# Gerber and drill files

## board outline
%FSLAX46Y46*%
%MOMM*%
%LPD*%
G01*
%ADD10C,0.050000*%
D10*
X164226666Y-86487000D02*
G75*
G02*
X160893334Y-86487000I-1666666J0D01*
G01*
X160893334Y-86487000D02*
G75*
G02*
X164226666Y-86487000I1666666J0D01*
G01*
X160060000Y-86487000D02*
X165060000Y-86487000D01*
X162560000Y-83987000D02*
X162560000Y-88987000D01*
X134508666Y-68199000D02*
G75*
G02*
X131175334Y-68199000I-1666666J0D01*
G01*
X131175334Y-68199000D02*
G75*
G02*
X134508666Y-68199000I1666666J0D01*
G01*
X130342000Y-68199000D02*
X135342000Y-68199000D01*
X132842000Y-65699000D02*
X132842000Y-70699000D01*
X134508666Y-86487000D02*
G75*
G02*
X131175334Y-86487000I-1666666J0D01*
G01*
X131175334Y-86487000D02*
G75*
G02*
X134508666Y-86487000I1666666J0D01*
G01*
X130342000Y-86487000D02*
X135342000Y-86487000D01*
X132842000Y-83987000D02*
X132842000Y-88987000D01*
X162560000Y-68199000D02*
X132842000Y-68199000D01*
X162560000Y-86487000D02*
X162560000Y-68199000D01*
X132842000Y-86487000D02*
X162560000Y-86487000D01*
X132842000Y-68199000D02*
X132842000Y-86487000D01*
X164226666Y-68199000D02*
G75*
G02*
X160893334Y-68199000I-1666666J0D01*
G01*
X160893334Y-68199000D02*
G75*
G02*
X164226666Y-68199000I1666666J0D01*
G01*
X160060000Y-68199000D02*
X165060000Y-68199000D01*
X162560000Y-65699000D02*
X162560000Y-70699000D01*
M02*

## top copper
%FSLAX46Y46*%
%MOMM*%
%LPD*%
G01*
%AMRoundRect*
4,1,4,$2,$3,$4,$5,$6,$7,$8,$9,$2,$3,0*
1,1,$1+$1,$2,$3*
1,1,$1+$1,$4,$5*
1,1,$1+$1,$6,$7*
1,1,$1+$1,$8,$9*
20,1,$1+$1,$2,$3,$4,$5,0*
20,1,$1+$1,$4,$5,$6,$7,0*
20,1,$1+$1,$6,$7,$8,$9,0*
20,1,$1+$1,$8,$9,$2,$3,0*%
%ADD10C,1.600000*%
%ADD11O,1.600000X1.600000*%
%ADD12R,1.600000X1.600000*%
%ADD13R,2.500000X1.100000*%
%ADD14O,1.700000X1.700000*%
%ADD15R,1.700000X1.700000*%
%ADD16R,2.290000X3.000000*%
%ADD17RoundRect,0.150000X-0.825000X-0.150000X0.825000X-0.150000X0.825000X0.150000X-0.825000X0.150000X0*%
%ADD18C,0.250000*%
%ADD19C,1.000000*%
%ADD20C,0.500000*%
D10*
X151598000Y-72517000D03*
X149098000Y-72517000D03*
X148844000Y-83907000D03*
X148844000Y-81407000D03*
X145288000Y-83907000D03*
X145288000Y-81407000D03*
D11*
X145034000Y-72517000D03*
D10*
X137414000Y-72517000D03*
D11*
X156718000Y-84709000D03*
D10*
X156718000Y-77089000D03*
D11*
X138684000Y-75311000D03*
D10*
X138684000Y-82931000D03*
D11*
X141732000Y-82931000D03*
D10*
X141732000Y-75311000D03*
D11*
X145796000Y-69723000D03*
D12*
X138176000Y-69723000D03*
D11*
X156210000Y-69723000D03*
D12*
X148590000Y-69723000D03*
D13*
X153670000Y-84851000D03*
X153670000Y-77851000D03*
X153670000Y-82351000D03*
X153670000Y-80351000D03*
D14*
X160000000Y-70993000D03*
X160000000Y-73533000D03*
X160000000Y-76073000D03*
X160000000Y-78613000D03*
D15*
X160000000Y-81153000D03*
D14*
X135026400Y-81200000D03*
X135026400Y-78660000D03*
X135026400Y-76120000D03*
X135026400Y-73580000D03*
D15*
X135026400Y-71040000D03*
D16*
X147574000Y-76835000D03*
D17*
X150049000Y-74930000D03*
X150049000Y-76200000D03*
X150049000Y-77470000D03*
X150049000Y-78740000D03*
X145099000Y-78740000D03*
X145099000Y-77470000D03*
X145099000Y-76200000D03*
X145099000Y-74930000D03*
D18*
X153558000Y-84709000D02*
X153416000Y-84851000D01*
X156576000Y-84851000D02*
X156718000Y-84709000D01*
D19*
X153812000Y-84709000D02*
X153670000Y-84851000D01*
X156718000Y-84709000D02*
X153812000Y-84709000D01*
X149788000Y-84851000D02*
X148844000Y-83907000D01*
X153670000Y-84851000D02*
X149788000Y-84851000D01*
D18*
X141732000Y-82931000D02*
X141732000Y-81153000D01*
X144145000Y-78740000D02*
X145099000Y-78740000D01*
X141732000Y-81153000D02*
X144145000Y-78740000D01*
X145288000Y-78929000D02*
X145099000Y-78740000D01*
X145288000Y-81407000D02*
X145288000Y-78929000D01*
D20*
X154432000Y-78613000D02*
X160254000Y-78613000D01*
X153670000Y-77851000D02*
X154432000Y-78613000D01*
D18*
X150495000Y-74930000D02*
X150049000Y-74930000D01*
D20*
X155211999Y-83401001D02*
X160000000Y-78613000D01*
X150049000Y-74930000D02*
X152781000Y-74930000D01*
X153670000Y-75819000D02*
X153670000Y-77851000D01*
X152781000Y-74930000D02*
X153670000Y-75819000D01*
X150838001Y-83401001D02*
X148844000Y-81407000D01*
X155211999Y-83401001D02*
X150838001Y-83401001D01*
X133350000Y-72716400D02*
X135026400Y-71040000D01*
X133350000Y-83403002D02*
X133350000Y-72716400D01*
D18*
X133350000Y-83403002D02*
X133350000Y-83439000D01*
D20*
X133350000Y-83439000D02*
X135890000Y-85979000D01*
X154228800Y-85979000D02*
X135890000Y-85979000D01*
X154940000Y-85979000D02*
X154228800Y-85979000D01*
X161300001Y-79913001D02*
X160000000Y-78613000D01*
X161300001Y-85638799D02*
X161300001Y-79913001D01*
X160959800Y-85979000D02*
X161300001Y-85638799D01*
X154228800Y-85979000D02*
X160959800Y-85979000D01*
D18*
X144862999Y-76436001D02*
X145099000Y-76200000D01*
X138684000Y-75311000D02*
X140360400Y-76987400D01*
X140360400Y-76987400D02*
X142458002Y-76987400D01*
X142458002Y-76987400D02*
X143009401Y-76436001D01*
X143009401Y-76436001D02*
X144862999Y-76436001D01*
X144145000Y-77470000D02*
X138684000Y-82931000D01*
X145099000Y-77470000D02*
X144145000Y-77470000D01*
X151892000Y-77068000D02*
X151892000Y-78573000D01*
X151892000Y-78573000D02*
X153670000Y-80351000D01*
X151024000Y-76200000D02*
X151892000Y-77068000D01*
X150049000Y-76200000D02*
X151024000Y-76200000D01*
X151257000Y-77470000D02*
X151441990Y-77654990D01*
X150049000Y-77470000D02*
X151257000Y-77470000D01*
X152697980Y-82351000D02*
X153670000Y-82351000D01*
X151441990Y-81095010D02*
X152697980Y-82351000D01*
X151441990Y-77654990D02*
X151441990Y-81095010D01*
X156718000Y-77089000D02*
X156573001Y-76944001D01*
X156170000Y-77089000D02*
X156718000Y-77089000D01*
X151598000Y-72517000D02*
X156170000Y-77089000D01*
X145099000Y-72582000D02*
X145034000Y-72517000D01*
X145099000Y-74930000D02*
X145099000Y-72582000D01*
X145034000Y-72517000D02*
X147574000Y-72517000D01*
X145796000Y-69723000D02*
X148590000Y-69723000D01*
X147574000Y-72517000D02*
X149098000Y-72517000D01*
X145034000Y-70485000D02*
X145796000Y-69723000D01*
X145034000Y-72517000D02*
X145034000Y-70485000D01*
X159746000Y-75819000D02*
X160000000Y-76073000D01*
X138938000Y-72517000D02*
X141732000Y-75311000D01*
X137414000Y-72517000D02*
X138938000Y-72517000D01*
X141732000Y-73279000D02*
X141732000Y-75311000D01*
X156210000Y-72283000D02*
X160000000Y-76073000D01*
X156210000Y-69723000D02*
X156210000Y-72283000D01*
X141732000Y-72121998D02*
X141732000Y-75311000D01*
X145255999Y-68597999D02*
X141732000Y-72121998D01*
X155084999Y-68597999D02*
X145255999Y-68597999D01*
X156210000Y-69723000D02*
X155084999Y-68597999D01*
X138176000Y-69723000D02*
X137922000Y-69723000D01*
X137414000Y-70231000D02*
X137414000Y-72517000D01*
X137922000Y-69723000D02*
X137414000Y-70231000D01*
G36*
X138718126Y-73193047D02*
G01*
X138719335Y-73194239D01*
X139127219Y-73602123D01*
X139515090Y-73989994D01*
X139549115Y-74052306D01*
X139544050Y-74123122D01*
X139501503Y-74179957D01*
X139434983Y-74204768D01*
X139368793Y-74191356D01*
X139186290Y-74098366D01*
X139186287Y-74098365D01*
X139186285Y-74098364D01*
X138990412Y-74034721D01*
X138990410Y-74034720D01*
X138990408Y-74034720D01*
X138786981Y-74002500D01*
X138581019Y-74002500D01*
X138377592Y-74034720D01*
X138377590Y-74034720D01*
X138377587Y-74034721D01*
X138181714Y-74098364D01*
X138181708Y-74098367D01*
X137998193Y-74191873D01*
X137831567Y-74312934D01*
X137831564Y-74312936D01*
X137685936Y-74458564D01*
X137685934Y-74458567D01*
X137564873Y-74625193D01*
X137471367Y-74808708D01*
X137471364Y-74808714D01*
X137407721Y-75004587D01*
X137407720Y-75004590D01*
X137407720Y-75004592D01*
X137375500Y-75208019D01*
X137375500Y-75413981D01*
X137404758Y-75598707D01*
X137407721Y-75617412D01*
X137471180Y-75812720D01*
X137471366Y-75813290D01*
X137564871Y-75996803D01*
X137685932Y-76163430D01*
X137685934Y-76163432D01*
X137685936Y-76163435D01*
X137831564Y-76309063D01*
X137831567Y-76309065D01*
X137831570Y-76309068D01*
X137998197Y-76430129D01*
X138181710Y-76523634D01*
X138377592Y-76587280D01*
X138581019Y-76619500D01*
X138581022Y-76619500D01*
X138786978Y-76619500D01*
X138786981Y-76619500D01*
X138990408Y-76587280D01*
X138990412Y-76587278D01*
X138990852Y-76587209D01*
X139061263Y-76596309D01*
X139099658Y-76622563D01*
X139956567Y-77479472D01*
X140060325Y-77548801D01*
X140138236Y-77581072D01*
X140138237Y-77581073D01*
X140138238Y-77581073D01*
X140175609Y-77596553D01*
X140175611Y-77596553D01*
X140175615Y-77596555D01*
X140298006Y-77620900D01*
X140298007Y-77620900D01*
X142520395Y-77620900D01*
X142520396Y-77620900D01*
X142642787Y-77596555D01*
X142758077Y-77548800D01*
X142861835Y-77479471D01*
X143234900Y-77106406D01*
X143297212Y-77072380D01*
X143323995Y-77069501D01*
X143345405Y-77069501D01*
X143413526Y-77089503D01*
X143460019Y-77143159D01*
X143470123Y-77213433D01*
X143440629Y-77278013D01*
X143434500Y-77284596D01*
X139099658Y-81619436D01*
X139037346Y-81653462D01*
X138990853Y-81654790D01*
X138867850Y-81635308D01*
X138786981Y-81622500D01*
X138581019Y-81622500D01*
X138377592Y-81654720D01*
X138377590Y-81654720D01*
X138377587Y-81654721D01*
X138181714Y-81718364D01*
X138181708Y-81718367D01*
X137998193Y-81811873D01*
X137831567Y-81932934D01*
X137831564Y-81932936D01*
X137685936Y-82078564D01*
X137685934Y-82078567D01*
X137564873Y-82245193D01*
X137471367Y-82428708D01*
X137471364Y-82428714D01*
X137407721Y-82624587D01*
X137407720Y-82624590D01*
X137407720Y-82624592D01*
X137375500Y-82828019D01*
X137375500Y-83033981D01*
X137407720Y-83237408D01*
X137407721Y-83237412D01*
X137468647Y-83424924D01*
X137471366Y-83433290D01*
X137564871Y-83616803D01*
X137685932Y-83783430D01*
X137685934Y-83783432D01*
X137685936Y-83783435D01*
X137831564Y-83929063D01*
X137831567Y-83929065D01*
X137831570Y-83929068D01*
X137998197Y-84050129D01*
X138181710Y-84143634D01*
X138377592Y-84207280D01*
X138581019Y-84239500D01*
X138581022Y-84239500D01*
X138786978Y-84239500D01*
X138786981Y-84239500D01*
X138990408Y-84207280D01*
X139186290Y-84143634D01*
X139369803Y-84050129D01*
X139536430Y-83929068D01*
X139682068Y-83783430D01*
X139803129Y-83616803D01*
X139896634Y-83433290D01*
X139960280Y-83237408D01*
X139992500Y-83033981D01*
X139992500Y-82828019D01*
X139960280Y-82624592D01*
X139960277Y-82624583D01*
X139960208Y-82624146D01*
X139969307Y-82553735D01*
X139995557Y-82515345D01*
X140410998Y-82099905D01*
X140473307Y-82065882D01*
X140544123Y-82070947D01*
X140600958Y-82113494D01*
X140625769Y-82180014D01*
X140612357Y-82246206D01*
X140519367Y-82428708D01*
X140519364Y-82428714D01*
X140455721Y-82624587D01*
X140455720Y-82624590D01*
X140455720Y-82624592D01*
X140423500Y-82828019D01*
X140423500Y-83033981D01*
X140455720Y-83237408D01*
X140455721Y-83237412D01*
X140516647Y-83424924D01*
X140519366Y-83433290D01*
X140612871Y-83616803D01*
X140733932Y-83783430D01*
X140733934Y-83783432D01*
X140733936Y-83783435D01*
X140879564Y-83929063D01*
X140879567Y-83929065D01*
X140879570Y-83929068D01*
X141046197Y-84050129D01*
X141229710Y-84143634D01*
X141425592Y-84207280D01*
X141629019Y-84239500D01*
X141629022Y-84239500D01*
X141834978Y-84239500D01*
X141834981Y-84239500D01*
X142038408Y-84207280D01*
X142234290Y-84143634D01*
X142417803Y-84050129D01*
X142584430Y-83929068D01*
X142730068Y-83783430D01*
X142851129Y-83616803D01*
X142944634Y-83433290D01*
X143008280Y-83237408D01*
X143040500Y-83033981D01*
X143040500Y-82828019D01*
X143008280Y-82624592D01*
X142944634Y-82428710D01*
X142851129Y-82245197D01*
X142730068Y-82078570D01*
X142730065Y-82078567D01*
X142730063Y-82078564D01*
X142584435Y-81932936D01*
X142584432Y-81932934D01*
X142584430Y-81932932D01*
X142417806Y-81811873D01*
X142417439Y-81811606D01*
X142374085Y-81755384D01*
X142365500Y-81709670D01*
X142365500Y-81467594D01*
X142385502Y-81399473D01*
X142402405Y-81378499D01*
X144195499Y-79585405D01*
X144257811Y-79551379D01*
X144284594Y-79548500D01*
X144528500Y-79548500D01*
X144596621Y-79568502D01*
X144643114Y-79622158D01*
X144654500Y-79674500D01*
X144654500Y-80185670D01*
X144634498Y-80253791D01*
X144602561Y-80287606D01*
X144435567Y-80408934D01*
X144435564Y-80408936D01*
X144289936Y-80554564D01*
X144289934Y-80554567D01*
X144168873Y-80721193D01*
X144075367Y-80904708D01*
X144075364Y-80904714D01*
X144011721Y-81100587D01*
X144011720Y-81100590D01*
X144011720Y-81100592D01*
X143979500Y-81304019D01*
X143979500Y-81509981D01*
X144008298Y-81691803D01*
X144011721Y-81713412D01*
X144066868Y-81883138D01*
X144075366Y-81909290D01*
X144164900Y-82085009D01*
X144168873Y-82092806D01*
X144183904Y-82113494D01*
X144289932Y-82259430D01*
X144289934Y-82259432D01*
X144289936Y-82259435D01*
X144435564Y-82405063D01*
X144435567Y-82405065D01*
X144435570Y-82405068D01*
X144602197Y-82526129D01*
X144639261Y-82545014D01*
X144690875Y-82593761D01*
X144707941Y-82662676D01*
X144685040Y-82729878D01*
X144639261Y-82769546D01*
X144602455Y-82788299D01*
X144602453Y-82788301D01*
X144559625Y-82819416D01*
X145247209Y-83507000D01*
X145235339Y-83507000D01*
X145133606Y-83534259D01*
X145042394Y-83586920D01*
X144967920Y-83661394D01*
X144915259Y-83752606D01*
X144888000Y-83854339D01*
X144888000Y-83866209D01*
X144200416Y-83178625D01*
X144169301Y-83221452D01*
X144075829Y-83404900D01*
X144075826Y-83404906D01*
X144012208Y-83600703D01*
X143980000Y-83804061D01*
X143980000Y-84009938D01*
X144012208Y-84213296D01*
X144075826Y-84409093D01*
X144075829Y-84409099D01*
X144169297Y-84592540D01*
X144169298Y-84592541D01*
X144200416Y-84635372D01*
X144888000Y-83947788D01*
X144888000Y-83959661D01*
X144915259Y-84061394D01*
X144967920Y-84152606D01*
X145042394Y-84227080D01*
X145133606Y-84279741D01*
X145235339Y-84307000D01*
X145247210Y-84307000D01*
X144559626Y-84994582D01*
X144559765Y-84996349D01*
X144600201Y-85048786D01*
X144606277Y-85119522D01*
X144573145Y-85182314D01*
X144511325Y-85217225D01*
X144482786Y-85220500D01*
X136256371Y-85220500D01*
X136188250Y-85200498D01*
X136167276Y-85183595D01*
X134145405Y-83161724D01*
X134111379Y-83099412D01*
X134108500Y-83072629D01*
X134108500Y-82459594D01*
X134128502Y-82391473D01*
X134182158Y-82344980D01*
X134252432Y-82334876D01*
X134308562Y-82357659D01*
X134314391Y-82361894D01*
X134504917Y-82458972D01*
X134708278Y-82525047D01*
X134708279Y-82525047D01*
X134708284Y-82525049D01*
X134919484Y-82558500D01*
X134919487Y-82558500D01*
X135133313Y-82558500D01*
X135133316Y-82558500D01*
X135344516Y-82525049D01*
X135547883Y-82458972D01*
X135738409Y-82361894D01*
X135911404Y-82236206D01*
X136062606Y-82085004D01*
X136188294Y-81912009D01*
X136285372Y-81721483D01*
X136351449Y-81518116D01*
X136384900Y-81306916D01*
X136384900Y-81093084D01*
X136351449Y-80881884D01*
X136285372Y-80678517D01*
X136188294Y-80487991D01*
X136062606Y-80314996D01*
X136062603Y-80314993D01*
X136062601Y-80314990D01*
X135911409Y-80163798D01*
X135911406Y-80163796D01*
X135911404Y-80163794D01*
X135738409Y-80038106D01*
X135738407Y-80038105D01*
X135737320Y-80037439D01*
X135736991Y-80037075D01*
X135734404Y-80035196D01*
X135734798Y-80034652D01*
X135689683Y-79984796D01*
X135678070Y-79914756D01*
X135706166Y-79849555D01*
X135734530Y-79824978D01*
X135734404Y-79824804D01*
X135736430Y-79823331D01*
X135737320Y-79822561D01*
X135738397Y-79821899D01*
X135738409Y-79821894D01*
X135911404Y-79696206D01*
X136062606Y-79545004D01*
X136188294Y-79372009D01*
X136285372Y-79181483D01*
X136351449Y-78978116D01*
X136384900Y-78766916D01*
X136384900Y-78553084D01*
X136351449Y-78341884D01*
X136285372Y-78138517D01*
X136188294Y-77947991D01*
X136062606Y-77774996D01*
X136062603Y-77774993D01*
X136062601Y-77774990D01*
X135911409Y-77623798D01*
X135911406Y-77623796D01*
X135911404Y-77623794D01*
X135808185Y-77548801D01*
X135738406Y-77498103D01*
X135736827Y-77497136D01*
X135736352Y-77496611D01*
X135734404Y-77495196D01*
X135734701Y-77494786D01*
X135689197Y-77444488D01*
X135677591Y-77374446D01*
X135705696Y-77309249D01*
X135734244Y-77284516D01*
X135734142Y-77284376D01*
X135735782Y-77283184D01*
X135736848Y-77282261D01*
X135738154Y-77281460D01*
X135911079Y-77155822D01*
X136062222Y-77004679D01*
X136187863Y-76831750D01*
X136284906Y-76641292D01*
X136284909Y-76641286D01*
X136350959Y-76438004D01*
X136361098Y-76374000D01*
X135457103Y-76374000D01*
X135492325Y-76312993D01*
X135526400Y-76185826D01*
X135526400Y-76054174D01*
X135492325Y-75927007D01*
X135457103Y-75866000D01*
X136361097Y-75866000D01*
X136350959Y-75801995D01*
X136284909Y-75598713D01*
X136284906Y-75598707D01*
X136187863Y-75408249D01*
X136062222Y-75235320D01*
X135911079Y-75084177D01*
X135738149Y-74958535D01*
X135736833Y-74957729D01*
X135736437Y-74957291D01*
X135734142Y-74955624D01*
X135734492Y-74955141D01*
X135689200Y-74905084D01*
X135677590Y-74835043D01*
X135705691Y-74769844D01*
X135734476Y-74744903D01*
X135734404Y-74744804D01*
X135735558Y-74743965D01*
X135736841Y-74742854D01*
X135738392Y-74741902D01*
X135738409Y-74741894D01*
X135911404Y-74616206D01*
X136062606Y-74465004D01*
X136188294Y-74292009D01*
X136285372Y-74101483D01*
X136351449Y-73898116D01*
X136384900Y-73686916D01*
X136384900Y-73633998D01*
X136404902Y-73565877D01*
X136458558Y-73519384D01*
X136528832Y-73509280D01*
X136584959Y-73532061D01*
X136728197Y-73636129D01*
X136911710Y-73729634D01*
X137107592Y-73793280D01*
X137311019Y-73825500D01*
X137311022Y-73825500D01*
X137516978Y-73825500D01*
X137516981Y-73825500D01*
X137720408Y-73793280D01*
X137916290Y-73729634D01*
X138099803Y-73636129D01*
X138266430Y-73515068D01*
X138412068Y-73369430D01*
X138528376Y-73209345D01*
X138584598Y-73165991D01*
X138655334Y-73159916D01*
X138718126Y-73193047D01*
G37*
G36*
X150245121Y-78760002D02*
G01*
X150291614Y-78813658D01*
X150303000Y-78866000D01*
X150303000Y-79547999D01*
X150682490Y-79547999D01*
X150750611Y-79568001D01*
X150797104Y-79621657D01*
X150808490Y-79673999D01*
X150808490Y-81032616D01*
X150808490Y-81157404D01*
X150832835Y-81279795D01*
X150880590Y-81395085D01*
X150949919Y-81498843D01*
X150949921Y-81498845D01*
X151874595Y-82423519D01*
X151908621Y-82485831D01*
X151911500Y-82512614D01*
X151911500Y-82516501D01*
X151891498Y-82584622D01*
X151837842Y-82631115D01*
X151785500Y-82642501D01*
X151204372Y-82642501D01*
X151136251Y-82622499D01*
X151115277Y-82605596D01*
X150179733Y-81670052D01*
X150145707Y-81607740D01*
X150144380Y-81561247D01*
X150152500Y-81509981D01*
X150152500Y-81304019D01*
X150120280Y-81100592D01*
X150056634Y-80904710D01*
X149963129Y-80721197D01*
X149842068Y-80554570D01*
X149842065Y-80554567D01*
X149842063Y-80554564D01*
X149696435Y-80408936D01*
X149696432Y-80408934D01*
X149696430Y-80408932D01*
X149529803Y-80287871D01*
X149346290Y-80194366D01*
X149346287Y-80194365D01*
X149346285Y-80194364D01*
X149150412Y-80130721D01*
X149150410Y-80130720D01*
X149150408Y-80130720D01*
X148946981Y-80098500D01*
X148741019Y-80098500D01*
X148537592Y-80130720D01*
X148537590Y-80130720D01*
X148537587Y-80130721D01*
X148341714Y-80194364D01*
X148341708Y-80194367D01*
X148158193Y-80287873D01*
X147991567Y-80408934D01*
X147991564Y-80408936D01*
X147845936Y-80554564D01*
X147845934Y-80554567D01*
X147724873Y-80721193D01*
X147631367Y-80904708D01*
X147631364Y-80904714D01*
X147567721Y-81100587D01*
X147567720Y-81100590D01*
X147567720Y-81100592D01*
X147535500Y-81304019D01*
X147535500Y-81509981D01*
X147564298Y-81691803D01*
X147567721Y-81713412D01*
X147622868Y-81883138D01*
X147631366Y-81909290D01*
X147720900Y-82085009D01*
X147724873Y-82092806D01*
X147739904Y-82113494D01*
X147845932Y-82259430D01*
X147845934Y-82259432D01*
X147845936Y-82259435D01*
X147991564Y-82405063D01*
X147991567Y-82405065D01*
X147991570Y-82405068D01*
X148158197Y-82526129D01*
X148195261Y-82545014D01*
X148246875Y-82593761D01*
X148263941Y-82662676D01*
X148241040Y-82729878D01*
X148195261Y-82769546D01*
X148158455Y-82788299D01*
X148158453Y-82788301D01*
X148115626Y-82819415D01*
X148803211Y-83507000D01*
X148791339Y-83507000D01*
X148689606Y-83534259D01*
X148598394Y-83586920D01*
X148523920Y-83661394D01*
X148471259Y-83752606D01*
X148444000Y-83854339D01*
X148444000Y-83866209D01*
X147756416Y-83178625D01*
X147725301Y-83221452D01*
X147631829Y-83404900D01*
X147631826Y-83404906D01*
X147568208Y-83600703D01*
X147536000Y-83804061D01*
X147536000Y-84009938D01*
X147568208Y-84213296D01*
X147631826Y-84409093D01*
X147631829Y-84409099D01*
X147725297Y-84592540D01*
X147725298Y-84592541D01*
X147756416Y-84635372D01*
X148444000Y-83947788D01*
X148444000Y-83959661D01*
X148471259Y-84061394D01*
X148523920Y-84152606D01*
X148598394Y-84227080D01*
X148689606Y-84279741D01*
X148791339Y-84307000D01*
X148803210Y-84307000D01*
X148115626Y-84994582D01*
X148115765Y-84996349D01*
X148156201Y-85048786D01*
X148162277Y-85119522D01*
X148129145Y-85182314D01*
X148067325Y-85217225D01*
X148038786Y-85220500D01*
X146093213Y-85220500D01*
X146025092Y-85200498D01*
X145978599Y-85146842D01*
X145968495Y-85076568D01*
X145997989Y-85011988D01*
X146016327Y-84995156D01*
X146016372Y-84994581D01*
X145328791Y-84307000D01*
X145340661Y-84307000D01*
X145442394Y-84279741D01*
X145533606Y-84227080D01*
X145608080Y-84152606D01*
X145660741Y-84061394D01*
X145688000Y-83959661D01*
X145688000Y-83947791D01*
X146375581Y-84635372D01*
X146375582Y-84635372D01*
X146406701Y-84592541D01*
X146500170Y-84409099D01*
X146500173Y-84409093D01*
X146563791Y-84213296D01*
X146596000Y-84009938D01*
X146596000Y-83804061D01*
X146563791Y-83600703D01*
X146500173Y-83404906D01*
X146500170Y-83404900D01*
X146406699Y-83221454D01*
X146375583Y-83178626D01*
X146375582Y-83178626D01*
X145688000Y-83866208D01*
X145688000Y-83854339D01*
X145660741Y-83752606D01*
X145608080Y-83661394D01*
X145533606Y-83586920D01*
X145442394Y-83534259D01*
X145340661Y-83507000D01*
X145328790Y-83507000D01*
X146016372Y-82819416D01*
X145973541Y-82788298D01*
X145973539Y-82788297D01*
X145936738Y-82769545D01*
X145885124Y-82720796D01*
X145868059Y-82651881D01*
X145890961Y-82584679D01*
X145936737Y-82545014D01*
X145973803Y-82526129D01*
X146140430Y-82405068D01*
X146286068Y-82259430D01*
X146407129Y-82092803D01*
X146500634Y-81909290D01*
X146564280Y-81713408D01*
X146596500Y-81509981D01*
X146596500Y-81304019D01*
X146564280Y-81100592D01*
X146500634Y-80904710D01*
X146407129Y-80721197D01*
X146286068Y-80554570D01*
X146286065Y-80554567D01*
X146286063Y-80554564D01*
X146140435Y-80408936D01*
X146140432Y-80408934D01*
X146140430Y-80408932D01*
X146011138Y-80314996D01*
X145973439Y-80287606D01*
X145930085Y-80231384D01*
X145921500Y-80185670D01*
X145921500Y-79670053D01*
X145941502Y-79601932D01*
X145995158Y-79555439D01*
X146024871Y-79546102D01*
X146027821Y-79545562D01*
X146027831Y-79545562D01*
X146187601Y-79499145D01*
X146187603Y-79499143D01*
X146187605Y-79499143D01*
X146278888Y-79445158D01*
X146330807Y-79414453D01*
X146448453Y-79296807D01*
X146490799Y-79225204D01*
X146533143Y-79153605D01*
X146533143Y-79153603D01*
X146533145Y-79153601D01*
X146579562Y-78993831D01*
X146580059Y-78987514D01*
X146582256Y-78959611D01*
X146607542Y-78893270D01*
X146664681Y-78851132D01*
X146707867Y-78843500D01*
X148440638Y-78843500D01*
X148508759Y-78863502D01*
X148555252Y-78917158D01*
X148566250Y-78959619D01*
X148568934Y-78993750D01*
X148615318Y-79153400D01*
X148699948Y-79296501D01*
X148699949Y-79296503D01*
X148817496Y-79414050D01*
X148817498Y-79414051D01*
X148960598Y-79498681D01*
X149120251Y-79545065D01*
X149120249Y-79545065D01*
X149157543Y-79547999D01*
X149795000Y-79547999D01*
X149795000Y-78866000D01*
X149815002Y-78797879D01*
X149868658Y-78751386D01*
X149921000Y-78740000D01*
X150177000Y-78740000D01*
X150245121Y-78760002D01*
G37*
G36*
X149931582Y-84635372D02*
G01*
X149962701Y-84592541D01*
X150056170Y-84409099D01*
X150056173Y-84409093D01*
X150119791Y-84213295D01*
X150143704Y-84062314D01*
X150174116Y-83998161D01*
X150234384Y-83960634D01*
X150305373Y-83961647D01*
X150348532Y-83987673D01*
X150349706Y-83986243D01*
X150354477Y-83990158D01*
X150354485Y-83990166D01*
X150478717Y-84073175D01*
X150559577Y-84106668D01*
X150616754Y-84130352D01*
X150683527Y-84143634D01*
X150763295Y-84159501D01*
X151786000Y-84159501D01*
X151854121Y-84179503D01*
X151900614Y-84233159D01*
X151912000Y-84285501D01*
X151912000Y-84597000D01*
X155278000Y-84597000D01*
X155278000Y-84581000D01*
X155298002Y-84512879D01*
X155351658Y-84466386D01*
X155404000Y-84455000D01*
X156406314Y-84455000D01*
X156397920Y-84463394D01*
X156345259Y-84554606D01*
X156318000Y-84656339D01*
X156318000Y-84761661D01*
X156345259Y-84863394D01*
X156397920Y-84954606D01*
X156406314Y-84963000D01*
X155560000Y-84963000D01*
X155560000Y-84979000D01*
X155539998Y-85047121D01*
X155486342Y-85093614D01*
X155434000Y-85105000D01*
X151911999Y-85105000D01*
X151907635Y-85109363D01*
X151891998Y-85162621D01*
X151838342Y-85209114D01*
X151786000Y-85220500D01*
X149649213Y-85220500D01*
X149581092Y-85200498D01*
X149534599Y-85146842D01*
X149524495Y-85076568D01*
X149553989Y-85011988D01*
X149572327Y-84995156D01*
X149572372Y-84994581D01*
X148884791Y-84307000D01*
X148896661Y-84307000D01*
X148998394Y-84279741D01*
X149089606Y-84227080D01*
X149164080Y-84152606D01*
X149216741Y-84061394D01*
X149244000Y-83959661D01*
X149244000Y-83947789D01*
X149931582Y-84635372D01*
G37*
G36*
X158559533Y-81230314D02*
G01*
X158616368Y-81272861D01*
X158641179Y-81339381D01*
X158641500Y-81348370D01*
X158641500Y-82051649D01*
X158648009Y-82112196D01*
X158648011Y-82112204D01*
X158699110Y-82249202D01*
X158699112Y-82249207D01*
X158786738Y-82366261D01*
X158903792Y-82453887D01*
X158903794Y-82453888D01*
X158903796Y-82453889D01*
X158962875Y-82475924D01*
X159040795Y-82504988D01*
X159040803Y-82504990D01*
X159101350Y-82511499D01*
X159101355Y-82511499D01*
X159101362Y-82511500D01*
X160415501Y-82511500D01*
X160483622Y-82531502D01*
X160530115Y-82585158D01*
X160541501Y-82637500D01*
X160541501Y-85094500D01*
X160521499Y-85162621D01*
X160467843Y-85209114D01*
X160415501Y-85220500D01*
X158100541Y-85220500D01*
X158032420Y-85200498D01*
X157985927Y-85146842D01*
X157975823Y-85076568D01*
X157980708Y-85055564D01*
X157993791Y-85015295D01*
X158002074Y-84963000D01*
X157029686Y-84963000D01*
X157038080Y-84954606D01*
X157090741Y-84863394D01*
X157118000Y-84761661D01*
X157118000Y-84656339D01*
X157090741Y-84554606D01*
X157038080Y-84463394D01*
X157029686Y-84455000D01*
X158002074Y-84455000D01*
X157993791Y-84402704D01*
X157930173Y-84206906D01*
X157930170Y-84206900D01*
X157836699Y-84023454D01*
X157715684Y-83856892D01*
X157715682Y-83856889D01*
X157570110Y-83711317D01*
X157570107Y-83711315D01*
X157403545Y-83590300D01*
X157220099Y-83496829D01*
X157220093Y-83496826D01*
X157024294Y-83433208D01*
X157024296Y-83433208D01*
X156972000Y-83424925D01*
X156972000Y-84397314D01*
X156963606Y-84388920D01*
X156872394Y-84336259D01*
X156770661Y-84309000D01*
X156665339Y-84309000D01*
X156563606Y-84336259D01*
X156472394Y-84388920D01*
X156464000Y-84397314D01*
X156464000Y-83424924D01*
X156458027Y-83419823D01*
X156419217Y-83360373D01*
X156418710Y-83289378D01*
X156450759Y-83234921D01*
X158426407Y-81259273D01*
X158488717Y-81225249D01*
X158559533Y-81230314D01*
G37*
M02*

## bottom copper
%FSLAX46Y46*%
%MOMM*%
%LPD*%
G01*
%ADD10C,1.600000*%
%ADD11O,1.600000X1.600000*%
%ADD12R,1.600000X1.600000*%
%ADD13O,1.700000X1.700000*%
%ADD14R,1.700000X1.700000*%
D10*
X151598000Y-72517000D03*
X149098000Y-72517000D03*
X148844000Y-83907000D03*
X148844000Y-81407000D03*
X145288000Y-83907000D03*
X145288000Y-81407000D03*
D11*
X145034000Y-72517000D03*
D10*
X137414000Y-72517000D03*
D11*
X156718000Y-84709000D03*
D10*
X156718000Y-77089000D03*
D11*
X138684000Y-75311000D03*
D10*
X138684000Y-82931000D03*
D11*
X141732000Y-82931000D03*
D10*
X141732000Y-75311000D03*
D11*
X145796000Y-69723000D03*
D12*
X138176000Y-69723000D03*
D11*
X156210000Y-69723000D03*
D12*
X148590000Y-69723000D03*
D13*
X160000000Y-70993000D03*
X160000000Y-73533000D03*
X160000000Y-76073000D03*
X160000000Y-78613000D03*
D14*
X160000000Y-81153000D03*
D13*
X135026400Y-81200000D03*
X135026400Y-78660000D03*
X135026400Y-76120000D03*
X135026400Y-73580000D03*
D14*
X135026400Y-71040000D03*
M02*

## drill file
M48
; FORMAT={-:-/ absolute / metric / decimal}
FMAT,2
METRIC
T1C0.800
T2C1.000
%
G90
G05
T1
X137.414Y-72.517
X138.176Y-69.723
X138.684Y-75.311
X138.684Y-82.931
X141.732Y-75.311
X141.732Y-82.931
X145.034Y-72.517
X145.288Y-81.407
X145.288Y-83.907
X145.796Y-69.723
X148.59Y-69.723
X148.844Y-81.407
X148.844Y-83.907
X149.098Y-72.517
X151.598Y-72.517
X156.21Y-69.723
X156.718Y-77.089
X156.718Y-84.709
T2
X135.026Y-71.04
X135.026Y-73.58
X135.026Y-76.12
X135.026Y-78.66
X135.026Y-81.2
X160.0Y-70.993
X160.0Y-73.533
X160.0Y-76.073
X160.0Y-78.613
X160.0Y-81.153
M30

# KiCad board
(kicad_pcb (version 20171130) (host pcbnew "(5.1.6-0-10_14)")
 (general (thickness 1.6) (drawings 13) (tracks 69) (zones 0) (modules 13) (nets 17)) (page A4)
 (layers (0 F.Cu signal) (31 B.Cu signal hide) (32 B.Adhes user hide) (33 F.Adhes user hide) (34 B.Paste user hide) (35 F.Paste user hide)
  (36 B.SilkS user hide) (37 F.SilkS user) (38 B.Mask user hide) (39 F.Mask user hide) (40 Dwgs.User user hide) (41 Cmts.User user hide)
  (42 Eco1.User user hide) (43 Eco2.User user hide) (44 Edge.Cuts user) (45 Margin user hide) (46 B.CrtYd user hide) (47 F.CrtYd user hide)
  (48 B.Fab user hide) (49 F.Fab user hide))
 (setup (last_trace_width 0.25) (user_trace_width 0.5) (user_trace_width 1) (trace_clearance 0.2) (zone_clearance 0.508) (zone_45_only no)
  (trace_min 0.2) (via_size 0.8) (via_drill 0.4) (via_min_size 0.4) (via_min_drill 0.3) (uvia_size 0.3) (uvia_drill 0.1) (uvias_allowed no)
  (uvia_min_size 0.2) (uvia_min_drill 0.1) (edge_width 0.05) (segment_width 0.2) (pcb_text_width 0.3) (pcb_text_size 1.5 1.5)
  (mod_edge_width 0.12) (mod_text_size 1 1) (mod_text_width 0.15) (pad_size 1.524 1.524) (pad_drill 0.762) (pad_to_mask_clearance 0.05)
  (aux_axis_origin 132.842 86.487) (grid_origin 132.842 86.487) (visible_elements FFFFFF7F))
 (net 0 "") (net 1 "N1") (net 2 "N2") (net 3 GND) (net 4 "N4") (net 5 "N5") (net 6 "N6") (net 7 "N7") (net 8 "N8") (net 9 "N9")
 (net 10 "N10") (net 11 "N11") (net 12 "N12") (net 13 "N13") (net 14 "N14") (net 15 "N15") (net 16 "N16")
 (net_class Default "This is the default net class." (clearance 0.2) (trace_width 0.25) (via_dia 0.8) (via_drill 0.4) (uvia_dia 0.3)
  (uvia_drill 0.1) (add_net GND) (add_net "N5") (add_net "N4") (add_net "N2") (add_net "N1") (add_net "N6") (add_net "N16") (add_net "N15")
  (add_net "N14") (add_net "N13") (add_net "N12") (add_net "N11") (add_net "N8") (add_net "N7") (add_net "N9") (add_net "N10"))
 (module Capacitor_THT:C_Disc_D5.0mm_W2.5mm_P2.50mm (layer F.Cu) (at 149.098 72.517)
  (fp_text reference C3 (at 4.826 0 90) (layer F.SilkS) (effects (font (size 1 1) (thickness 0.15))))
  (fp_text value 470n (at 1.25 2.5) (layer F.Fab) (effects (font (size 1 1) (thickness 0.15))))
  (pad 2 thru_hole circle (at 2.5 0) (size 1.6 1.6) (drill 0.8) (layers *.Cu *.Mask) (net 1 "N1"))
  (pad 1 thru_hole circle (at 0 0) (size 1.6 1.6) (drill 0.8) (layers *.Cu *.Mask) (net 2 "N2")))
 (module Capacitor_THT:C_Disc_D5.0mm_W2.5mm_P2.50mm (layer F.Cu) (at 148.844 81.407 270)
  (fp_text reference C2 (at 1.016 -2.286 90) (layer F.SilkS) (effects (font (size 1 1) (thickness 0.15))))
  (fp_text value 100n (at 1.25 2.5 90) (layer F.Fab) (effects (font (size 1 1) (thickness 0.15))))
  (pad 2 thru_hole circle (at 2.5 0 270) (size 1.6 1.6) (drill 0.8) (layers *.Cu *.Mask) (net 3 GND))
  (pad 1 thru_hole circle (at 0 0 270) (size 1.6 1.6) (drill 0.8) (layers *.Cu *.Mask) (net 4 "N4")))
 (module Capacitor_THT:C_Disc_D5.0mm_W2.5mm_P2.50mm (layer F.Cu) (at 145.288 81.407 270)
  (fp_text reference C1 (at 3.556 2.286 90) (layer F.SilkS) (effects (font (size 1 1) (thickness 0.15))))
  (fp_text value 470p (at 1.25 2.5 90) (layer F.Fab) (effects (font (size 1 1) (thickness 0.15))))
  (pad 2 thru_hole circle (at 2.5 0 270) (size 1.6 1.6) (drill 0.8) (layers *.Cu *.Mask) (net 3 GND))
  (pad 1 thru_hole circle (at 0 0 270) (size 1.6 1.6) (drill 0.8) (layers *.Cu *.Mask) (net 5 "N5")))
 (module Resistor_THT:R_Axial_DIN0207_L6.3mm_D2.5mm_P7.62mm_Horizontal (layer F.Cu) (at 137.414 72.517)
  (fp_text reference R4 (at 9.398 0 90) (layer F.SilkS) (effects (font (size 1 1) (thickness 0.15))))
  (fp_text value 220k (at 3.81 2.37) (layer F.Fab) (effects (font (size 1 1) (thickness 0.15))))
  (pad 2 thru_hole oval (at 7.62 0) (size 1.6 1.6) (drill 0.8) (layers *.Cu *.Mask) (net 2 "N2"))
  (pad 1 thru_hole circle (at 0 0) (size 1.6 1.6) (drill 0.8) (layers *.Cu *.Mask) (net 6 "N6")))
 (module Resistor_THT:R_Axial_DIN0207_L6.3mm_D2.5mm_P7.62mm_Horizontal (layer F.Cu) (at 156.718 77.089 270)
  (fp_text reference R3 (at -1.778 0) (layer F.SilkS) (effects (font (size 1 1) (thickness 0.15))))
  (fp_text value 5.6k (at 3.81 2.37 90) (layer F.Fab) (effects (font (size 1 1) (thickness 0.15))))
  (pad 2 thru_hole oval (at 7.62 0 270) (size 1.6 1.6) (drill 0.8) (layers *.Cu *.Mask) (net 3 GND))
  (pad 1 thru_hole circle (at 0 0 270) (size 1.6 1.6) (drill 0.8) (layers *.Cu *.Mask) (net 1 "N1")))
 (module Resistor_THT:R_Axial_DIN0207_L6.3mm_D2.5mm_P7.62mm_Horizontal (layer F.Cu) (at 138.684 82.931 90)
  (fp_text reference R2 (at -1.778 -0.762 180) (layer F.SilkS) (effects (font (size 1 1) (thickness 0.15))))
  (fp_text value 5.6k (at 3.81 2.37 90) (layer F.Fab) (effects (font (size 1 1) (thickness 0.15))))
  (pad 2 thru_hole oval (at 7.62 0 90) (size 1.6 1.6) (drill 0.8) (layers *.Cu *.Mask) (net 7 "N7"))
  (pad 1 thru_hole circle (at 0 0 90) (size 1.6 1.6) (drill 0.8) (layers *.Cu *.Mask) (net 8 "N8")))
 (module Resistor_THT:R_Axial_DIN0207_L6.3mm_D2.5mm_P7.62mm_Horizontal (layer F.Cu) (at 141.732 75.311 270)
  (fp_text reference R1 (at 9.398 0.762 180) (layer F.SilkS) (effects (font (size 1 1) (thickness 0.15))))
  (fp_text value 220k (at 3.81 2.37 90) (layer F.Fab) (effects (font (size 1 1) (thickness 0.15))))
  (pad 2 thru_hole oval (at 7.62 0 270) (size 1.6 1.6) (drill 0.8) (layers *.Cu *.Mask) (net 5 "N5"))
  (pad 1 thru_hole circle (at 0 0 270) (size 1.6 1.6) (drill 0.8) (layers *.Cu *.Mask) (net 6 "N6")))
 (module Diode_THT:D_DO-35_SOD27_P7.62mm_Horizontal (layer F.Cu) (at 138.176 69.723)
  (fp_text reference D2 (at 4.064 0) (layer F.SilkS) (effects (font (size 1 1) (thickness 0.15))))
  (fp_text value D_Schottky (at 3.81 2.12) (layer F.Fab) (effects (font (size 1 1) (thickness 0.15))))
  (pad 2 thru_hole oval (at 7.62 0) (size 1.6 1.6) (drill 0.8) (layers *.Cu *.Mask) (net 2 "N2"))
  (pad 1 thru_hole rect (at 0 0) (size 1.6 1.6) (drill 0.8) (layers *.Cu *.Mask) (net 6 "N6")))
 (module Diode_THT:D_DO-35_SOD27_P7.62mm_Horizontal (layer F.Cu) (at 148.59 69.723)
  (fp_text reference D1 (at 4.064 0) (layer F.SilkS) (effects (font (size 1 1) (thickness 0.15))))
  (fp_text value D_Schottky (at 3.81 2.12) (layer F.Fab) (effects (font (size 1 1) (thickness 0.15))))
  (pad 2 thru_hole oval (at 7.62 0) (size 1.6 1.6) (drill 0.8) (layers *.Cu *.Mask) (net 6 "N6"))
  (pad 1 thru_hole rect (at 0 0) (size 1.6 1.6) (drill 0.8) (layers *.Cu *.Mask) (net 2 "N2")))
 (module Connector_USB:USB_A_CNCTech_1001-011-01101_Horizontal (layer F.Cu) (at 163.32 81.351)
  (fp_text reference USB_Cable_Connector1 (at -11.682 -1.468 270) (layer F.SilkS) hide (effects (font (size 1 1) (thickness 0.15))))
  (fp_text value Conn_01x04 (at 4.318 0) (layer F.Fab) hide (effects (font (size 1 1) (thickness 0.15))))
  (pad 4 smd rect (at -9.65 3.5) (size 2.5 1.1) (layers F.Cu F.Paste F.Mask) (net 3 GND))
  (pad 1 smd rect (at -9.65 -3.5) (size 2.5 1.1) (layers F.Cu F.Paste F.Mask) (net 4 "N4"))
  (pad 3 smd rect (at -9.65 1) (size 2.5 1.1) (layers F.Cu F.Paste F.Mask) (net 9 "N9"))
  (pad 2 smd rect (at -9.65 -1) (size 2.5 1.1) (layers F.Cu F.Paste F.Mask) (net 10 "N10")))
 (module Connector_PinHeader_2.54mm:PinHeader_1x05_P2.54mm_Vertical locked (layer B.Cu) (at 160 81.153)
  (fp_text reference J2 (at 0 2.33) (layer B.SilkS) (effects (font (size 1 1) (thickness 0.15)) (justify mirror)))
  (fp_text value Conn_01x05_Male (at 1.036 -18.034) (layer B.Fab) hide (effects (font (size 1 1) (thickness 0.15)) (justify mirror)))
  (pad 5 thru_hole oval (at 0 -10.16) (size 1.7 1.7) (drill 1) (layers *.Cu *.Mask) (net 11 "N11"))
  (pad 4 thru_hole oval (at 0 -7.62) (size 1.7 1.7) (drill 1) (layers *.Cu *.Mask) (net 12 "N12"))
  (pad 3 thru_hole oval (at 0 -5.08) (size 1.7 1.7) (drill 1) (layers *.Cu *.Mask) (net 6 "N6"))
  (pad 2 thru_hole oval (at 0 -2.54) (size 1.7 1.7) (drill 1) (layers *.Cu *.Mask) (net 4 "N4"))
  (pad 1 thru_hole rect (at 0 0) (size 1.7 1.7) (drill 1) (layers *.Cu *.Mask) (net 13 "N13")))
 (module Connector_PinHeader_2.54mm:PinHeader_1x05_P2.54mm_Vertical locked (layer B.Cu) (at 135.0264 71.04 180)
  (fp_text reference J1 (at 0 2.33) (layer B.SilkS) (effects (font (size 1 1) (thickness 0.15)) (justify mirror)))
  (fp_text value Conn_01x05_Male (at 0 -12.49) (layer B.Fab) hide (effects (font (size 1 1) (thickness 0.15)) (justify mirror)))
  (pad 5 thru_hole oval (at 0 -10.16 180) (size 1.7 1.7) (drill 1) (layers *.Cu *.Mask) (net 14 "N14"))
  (pad 4 thru_hole oval (at 0 -7.62 180) (size 1.7 1.7) (drill 1) (layers *.Cu *.Mask) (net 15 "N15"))
  (pad 3 thru_hole oval (at 0 -5.08 180) (size 1.7 1.7) (drill 1) (layers *.Cu *.Mask) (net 3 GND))
  (pad 2 thru_hole oval (at 0 -2.54 180) (size 1.7 1.7) (drill 1) (layers *.Cu *.Mask) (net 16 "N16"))
  (pad 1 thru_hole rect (at 0 0 180) (size 1.7 1.7) (drill 1) (layers *.Cu *.Mask) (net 4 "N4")))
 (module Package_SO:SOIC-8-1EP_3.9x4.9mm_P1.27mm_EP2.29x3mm (layer F.Cu) (at 147.574 76.835)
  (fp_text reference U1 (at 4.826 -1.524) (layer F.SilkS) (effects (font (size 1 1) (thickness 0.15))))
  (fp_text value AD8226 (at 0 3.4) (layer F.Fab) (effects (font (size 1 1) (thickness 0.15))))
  (pad "" smd roundrect (at 0.57 0.75) (size 0.92 1.21) (layers F.Paste) (roundrect_rratio 0.25))
  (pad "" smd roundrect (at 0.57 -0.75) (size 0.92 1.21) (layers F.Paste) (roundrect_rratio 0.25))
  (pad "" smd roundrect (at -0.57 0.75) (size 0.92 1.21) (layers F.Paste) (roundrect_rratio 0.25))
  (pad "" smd roundrect (at -0.57 -0.75) (size 0.92 1.21) (layers F.Paste) (roundrect_rratio 0.25))
  (pad 9 smd rect (at 0 0) (size 2.29 3) (layers F.Cu F.Mask))
  (pad 8 smd roundrect (at 2.475 -1.905) (size 1.95 0.6) (layers F.Cu F.Paste F.Mask) (roundrect_rratio 0.25) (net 4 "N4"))
  (pad 7 smd roundrect (at 2.475 -0.635) (size 1.95 0.6) (layers F.Cu F.Paste F.Mask) (roundrect_rratio 0.25) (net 10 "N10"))
  (pad 6 smd roundrect (at 2.475 0.635) (size 1.95 0.6) (layers F.Cu F.Paste F.Mask) (roundrect_rratio 0.25) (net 9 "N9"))
  (pad 5 smd roundrect (at 2.475 1.905) (size 1.95 0.6) (layers F.Cu F.Paste F.Mask) (roundrect_rratio 0.25) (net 3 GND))
  (pad 4 smd roundrect (at -2.475 1.905) (size 1.95 0.6) (layers F.Cu F.Paste F.Mask) (roundrect_rratio 0.25) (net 5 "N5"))
  (pad 3 smd roundrect (at -2.475 0.635) (size 1.95 0.6) (layers F.Cu F.Paste F.Mask) (roundrect_rratio 0.25) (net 8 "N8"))
  (pad 2 smd roundrect (at -2.475 -0.635) (size 1.95 0.6) (layers F.Cu F.Paste F.Mask) (roundrect_rratio 0.25) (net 7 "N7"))
  (pad 1 smd roundrect (at -2.475 -1.905) (size 1.95 0.6) (layers F.Cu F.Paste F.Mask) (roundrect_rratio 0.25) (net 2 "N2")))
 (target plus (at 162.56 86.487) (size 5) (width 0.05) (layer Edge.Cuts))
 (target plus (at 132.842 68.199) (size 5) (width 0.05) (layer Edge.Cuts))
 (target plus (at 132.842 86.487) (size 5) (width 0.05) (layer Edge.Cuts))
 (gr_line (start 162.56 68.199) (end 132.842 68.199) (layer Edge.Cuts) (width 0.05))
 (gr_line (start 162.56 86.487) (end 162.56 68.199) (layer Edge.Cuts) (width 0.05))
 (gr_line (start 132.842 86.487) (end 162.56 86.487) (layer Edge.Cuts) (width 0.05))
 (gr_line (start 132.842 68.199) (end 132.842 86.487) (layer Edge.Cuts) (width 0.05))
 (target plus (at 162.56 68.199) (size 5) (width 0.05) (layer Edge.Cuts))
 (segment (start 153.558 84.709) (end 153.416 84.851) (width 0.25) (layer F.Cu) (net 3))
 (segment (start 156.576 84.851) (end 156.718 84.709) (width 0.25) (layer F.Cu) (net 3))
 (segment (start 153.812 84.709) (end 153.67 84.851) (width 1) (layer F.Cu) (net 3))
 (segment (start 156.718 84.709) (end 153.812 84.709) (width 1) (layer F.Cu) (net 3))
 (segment (start 149.788 84.851) (end 148.844 83.907) (width 1) (layer F.Cu) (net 3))
 (segment (start 153.67 84.851) (end 149.788 84.851) (width 1) (layer F.Cu) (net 3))
 (segment (start 141.732 82.931) (end 141.732 81.153) (width 0.25) (layer F.Cu) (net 5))
 (segment (start 144.145 78.74) (end 145.099 78.74) (width 0.25) (layer F.Cu) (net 5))
 (segment (start 141.732 81.153) (end 144.145 78.74) (width 0.25) (layer F.Cu) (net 5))
 (segment (start 145.288 78.929) (end 145.099 78.74) (width 0.25) (layer F.Cu) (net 5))
 (segment (start 145.288 81.407) (end 145.288 78.929) (width 0.25) (layer F.Cu) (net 5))
 (segment (start 154.432 78.613) (end 160.254 78.613) (width 0.5) (layer F.Cu) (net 4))
 (segment (start 153.67 77.851) (end 154.432 78.613) (width 0.5) (layer F.Cu) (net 4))
 (segment (start 150.495 74.93) (end 150.049 74.93) (width 0.25) (layer F.Cu) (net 4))
 (segment (start 155.211999 83.401001) (end 160 78.613) (width 0.5) (layer F.Cu) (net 4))
 (segment (start 150.049 74.93) (end 152.781 74.93) (width 0.5) (layer F.Cu) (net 4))
 (segment (start 153.67 75.819) (end 153.67 77.851) (width 0.5) (layer F.Cu) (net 4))
 (segment (start 152.781 74.93) (end 153.67 75.819) (width 0.5) (layer F.Cu) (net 4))
 (segment (start 150.838001 83.401001) (end 148.844 81.407) (width 0.5) (layer F.Cu) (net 4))
 (segment (start 155.211999 83.401001) (end 150.838001 83.401001) (width 0.5) (layer F.Cu) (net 4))
 (segment (start 133.35 72.7164) (end 135.0264 71.04) (width 0.5) (layer F.Cu) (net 4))
 (segment (start 133.35 83.403002) (end 133.35 72.7164) (width 0.5) (layer F.Cu) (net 4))
 (segment (start 133.35 83.403002) (end 133.35 83.439) (width 0.25) (layer F.Cu) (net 4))
 (segment (start 133.35 83.439) (end 135.89 85.979) (width 0.5) (layer F.Cu) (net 4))
 (segment (start 154.2288 85.979) (end 135.89 85.979) (width 0.5) (layer F.Cu) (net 4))
 (segment (start 154.94 85.979) (end 154.2288 85.979) (width 0.5) (layer F.Cu) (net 4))
 (segment (start 161.300001 79.913001) (end 160 78.613) (width 0.5) (layer F.Cu) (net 4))
 (segment (start 161.300001 85.638799) (end 161.300001 79.913001) (width 0.5) (layer F.Cu) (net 4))
 (segment (start 160.9598 85.979) (end 161.300001 85.638799) (width 0.5) (layer F.Cu) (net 4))
 (segment (start 154.2288 85.979) (end 160.9598 85.979) (width 0.5) (layer F.Cu) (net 4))
 (segment (start 144.862999 76.436001) (end 145.099 76.2) (width 0.25) (layer F.Cu) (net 7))
 (segment (start 138.684 75.311) (end 140.3604 76.9874) (width 0.25) (layer F.Cu) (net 7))
 (segment (start 140.3604 76.9874) (end 142.458002 76.9874) (width 0.25) (layer F.Cu) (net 7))
 (segment (start 142.458002 76.9874) (end 143.009401 76.436001) (width 0.25) (layer F.Cu) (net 7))
 (segment (start 143.009401 76.436001) (end 144.862999 76.436001) (width 0.25) (layer F.Cu) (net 7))
 (segment (start 144.145 77.47) (end 138.684 82.931) (width 0.25) (layer F.Cu) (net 8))
 (segment (start 145.099 77.47) (end 144.145 77.47) (width 0.25) (layer F.Cu) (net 8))
 (segment (start 151.892 77.068) (end 151.892 78.573) (width 0.25) (layer F.Cu) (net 10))
 (segment (start 151.892 78.573) (end 153.67 80.351) (width 0.25) (layer F.Cu) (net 10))
 (segment (start 151.024 76.2) (end 151.892 77.068) (width 0.25) (layer F.Cu) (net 10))
 (segment (start 150.049 76.2) (end 151.024 76.2) (width 0.25) (layer F.Cu) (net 10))
 (segment (start 151.257 77.47) (end 151.44199 77.65499) (width 0.25) (layer F.Cu) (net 9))
 (segment (start 150.049 77.47) (end 151.257 77.47) (width 0.25) (layer F.Cu) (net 9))
 (segment (start 152.69798 82.351) (end 153.67 82.351) (width 0.25) (layer F.Cu) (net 9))
 (segment (start 151.44199 81.09501) (end 152.69798 82.351) (width 0.25) (layer F.Cu) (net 9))
 (segment (start 151.44199 77.65499) (end 151.44199 81.09501) (width 0.25) (layer F.Cu) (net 9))
 (segment (start 156.718 77.089) (end 156.573001 76.944001) (width 0.25) (layer F.Cu) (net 1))
 (segment (start 156.17 77.089) (end 156.718 77.089) (width 0.25) (layer F.Cu) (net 1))
 (segment (start 151.598 72.517) (end 156.17 77.089) (width 0.25) (layer F.Cu) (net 1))
 (segment (start 145.099 72.582) (end 145.034 72.517) (width 0.25) (layer F.Cu) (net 2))
 (segment (start 145.099 74.93) (end 145.099 72.582) (width 0.25) (layer F.Cu) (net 2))
 (segment (start 145.034 72.517) (end 147.574 72.517) (width 0.25) (layer F.Cu) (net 2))
 (segment (start 145.796 69.723) (end 148.59 69.723) (width 0.25) (layer F.Cu) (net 2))
 (segment (start 147.574 72.517) (end 149.098 72.517) (width 0.25) (layer F.Cu) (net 2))
 (segment (start 145.034 70.485) (end 145.796 69.723) (width 0.25) (layer F.Cu) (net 2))
 (segment (start 145.034 72.517) (end 145.034 70.485) (width 0.25) (layer F.Cu) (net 2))
 (segment (start 159.746 75.819) (end 160 76.073) (width 0.25) (layer F.Cu) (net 6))
 (segment (start 138.938 72.517) (end 141.732 75.311) (width 0.25) (layer F.Cu) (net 6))
 (segment (start 137.414 72.517) (end 138.938 72.517) (width 0.25) (layer F.Cu) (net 6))
 (segment (start 141.732 73.279) (end 141.732 75.311) (width 0.25) (layer F.Cu) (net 6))
 (segment (start 156.21 72.283) (end 160 76.073) (width 0.25) (layer F.Cu) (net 6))
 (segment (start 156.21 69.723) (end 156.21 72.283) (width 0.25) (layer F.Cu) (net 6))
 (segment (start 141.732 72.121998) (end 141.732 75.311) (width 0.25) (layer F.Cu) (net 6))
 (segment (start 145.255999 68.597999) (end 141.732 72.121998) (width 0.25) (layer F.Cu) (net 6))
 (segment (start 155.084999 68.597999) (end 145.255999 68.597999) (width 0.25) (layer F.Cu) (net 6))
 (segment (start 156.21 69.723) (end 155.084999 68.597999) (width 0.25) (layer F.Cu) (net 6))
 (segment (start 138.176 69.723) (end 137.922 69.723) (width 0.25) (layer F.Cu) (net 6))
 (segment (start 137.414 70.231) (end 137.414 72.517) (width 0.25) (layer F.Cu) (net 6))
 (segment (start 137.922 69.723) (end 137.414 70.231) (width 0.25) (layer F.Cu) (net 6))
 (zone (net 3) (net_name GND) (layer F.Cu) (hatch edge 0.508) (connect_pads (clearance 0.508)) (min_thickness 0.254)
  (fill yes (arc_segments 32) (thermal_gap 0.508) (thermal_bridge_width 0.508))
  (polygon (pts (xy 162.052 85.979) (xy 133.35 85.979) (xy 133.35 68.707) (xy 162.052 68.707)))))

